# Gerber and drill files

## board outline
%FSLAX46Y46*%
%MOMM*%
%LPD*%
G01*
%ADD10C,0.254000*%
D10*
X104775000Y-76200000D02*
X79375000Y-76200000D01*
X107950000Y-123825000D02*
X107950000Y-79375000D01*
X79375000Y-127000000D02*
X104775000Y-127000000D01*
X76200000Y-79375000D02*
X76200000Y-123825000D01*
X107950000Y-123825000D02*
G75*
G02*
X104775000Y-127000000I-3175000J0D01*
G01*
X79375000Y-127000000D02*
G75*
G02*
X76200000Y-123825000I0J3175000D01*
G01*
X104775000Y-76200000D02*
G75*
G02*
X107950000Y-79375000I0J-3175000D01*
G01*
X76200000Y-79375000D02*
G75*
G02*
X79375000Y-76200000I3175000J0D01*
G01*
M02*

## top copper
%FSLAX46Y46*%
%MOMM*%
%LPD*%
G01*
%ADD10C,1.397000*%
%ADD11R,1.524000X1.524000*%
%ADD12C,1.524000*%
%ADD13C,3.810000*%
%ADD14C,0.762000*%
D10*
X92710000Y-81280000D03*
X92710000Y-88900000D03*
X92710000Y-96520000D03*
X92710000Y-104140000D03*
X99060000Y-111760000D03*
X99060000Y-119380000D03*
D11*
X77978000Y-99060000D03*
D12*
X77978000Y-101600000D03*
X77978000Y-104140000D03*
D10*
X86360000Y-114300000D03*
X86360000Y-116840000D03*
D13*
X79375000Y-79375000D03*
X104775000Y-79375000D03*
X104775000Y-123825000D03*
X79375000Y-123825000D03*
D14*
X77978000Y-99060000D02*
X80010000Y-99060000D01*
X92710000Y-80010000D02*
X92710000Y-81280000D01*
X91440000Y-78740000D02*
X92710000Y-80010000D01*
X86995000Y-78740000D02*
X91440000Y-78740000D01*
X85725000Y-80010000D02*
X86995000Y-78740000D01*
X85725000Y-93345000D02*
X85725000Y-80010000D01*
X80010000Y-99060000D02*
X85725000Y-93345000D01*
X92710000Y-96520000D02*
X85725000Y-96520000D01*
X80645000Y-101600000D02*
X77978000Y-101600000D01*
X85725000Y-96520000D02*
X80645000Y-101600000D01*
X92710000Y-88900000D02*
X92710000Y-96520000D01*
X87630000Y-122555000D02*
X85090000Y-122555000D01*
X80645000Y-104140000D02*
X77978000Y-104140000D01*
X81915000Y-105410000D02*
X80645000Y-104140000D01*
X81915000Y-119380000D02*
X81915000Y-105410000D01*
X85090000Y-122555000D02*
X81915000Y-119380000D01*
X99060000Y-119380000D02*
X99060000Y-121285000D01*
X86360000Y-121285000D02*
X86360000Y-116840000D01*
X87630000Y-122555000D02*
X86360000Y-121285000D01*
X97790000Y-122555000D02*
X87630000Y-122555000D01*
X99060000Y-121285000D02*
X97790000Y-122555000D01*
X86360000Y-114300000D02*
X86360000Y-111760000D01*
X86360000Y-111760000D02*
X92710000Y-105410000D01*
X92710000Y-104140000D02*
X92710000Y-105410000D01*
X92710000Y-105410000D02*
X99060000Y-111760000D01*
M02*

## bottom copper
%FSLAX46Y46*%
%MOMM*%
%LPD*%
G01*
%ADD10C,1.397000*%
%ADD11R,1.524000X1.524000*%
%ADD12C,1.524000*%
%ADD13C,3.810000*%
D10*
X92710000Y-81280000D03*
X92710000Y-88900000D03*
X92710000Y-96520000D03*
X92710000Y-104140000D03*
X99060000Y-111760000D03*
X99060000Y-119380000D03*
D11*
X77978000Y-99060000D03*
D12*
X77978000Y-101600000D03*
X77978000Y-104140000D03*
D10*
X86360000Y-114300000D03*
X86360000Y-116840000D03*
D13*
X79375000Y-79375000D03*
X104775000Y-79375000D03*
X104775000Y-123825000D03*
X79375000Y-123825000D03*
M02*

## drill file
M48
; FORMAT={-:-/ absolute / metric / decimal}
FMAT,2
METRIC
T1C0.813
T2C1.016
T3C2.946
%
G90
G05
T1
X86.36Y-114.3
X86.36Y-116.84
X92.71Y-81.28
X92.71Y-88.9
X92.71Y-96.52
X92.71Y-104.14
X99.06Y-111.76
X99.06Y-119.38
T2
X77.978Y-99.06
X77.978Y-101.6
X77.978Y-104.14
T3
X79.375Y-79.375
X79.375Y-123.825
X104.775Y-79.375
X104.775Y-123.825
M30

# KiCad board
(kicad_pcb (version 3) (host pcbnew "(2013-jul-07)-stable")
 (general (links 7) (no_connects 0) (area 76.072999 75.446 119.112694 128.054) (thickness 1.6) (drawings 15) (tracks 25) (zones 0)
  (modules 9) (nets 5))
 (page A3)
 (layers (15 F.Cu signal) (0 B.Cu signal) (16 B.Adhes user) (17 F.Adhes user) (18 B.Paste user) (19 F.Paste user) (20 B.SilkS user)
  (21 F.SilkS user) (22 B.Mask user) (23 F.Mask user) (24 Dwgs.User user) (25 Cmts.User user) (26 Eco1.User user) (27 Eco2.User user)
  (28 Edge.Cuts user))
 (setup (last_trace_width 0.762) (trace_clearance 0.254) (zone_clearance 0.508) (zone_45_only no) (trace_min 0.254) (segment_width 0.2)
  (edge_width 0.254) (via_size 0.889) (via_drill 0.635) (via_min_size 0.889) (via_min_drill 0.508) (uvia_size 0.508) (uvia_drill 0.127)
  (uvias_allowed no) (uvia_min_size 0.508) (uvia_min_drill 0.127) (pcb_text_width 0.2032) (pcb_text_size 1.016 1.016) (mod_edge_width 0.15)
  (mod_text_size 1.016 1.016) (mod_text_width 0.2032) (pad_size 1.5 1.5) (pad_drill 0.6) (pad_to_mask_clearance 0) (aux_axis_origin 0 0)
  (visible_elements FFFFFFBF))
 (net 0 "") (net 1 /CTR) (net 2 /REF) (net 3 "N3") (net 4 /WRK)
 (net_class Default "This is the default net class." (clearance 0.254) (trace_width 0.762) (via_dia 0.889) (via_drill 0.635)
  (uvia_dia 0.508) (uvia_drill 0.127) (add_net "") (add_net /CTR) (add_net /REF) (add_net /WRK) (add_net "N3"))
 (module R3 (layer F.Cu) (at 92.71 85.09 270) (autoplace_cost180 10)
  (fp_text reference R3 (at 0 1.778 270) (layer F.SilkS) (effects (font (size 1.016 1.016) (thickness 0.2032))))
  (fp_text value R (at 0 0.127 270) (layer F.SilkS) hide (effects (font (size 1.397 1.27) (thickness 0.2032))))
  (pad 1 thru_hole circle (at -3.81 0 270) (size 1.397 1.397) (drill 0.8128) (layers *.Cu *.Mask F.SilkS) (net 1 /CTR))
  (pad 2 thru_hole circle (at 3.81 0 270) (size 1.397 1.397) (drill 0.8128) (layers *.Cu *.Mask F.SilkS) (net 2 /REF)))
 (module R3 (layer F.Cu) (at 92.71 100.33 270) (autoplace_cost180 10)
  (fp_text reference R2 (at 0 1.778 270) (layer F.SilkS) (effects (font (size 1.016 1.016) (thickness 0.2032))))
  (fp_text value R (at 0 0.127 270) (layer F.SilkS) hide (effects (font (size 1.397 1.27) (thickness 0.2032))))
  (pad 1 thru_hole circle (at -3.81 0 270) (size 1.397 1.397) (drill 0.8128) (layers *.Cu *.Mask F.SilkS) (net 2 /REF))
  (pad 2 thru_hole circle (at 3.81 0 270) (size 1.397 1.397) (drill 0.8128) (layers *.Cu *.Mask F.SilkS) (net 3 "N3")))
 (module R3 (layer F.Cu) (at 99.06 115.57 270) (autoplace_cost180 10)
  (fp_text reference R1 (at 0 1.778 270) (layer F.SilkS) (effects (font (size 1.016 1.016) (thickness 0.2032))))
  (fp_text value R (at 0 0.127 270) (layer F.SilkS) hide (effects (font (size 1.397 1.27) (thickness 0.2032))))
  (pad 1 thru_hole circle (at -3.81 0 270) (size 1.397 1.397) (drill 0.8128) (layers *.Cu *.Mask F.SilkS) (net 3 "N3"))
  (pad 2 thru_hole circle (at 3.81 0 270) (size 1.397 1.397) (drill 0.8128) (layers *.Cu *.Mask F.SilkS) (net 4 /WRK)))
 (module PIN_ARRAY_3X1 (layer F.Cu) (at 77.978 101.6 270)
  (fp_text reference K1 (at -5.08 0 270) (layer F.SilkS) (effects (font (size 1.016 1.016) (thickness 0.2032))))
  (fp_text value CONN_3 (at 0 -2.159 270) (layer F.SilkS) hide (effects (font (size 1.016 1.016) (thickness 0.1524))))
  (pad 1 thru_hole rect (at -2.54 0 270) (size 1.524 1.524) (drill 1.016) (layers *.Cu *.Mask F.SilkS) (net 1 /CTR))
  (pad 2 thru_hole circle (at 0 0 270) (size 1.524 1.524) (drill 1.016) (layers *.Cu *.Mask F.SilkS) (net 2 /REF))
  (pad 3 thru_hole circle (at 2.54 0 270) (size 1.524 1.524) (drill 1.016) (layers *.Cu *.Mask F.SilkS) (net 4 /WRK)))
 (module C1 (layer F.Cu) (at 86.36 115.57 270)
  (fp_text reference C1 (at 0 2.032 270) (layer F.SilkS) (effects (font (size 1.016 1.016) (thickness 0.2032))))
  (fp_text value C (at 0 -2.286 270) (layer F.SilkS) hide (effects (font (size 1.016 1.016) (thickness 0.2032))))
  (pad 1 thru_hole circle (at -1.27 0 270) (size 1.397 1.397) (drill 0.8128) (layers *.Cu *.Mask F.SilkS) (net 3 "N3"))
  (pad 2 thru_hole circle (at 1.27 0 270) (size 1.397 1.397) (drill 0.8128) (layers *.Cu *.Mask F.SilkS) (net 4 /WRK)))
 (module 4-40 (layer F.Cu) (at 79.375 79.375)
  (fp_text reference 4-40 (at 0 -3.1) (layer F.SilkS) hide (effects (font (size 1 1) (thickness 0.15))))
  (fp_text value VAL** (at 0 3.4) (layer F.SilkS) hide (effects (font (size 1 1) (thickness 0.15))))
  (pad "" thru_hole circle (at 0 0) (size 3.81 3.81) (drill 2.9464) (layers *.Cu *.Mask F.SilkS)))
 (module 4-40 (layer F.Cu) (at 104.775 79.375)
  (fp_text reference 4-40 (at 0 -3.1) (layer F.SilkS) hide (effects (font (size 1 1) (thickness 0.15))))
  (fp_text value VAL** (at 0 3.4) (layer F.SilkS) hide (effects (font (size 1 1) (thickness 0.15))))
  (pad "" thru_hole circle (at 0 0) (size 3.81 3.81) (drill 2.9464) (layers *.Cu *.Mask F.SilkS)))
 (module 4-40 (layer F.Cu) (at 104.775 123.825)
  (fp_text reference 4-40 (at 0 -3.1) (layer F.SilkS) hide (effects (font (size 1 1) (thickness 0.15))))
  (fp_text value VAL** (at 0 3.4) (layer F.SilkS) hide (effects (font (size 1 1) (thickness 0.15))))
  (pad "" thru_hole circle (at 0 0) (size 3.81 3.81) (drill 2.9464) (layers *.Cu *.Mask F.SilkS)))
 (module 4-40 (layer F.Cu) (at 79.375 123.825)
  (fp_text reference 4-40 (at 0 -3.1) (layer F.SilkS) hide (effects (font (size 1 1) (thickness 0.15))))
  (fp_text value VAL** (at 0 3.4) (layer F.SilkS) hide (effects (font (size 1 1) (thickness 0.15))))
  (pad "" thru_hole circle (at 0 0) (size 3.81 3.81) (drill 2.9464) (layers *.Cu *.Mask F.SilkS)))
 (gr_line (start 104.775 76.2) (end 79.375 76.2) (angle 90) (layer Edge.Cuts) (width 0.254))
 (gr_line (start 107.95 123.825) (end 107.95 79.375) (angle 90) (layer Edge.Cuts) (width 0.254))
 (gr_line (start 79.375 127) (end 104.775 127) (angle 90) (layer Edge.Cuts) (width 0.254))
 (gr_line (start 76.2 79.375) (end 76.2 123.825) (angle 90) (layer Edge.Cuts) (width 0.254))
 (gr_arc (start 104.775 123.825) (end 107.95 123.825) (angle 90) (layer Edge.Cuts) (width 0.254))
 (gr_arc (start 79.375 123.825) (end 79.375 127) (angle 90) (layer Edge.Cuts) (width 0.254))
 (gr_arc (start 104.775 79.375) (end 104.775 76.2) (angle 90) (layer Edge.Cuts) (width 0.254))
 (gr_arc (start 79.375 79.375) (end 76.2 79.375) (angle 90) (layer Edge.Cuts) (width 0.254))
 (segment (start 77.978 99.06) (end 80.01 99.06) (width 0.762) (layer F.Cu) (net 1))
 (segment (start 92.71 80.01) (end 92.71 81.28) (width 0.762) (layer F.Cu) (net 1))
 (segment (start 91.44 78.74) (end 92.71 80.01) (width 0.762) (layer F.Cu) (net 1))
 (segment (start 86.995 78.74) (end 91.44 78.74) (width 0.762) (layer F.Cu) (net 1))
 (segment (start 85.725 80.01) (end 86.995 78.74) (width 0.762) (layer F.Cu) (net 1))
 (segment (start 85.725 93.345) (end 85.725 80.01) (width 0.762) (layer F.Cu) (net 1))
 (segment (start 80.01 99.06) (end 85.725 93.345) (width 0.762) (layer F.Cu) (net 1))
 (segment (start 92.71 96.52) (end 85.725 96.52) (width 0.762) (layer F.Cu) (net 2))
 (segment (start 80.645 101.6) (end 77.978 101.6) (width 0.762) (layer F.Cu) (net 2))
 (segment (start 85.725 96.52) (end 80.645 101.6) (width 0.762) (layer F.Cu) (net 2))
 (segment (start 92.71 88.9) (end 92.71 96.52) (width 0.762) (layer F.Cu) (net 2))
 (segment (start 87.63 122.555) (end 85.09 122.555) (width 0.762) (layer F.Cu) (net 4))
 (segment (start 80.645 104.14) (end 77.978 104.14) (width 0.762) (layer F.Cu) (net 4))
 (segment (start 81.915 105.41) (end 80.645 104.14) (width 0.762) (layer F.Cu) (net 4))
 (segment (start 81.915 119.38) (end 81.915 105.41) (width 0.762) (layer F.Cu) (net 4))
 (segment (start 85.09 122.555) (end 81.915 119.38) (width 0.762) (layer F.Cu) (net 4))
 (segment (start 99.06 119.38) (end 99.06 121.285) (width 0.762) (layer F.Cu) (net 4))
 (segment (start 86.36 121.285) (end 86.36 116.84) (width 0.762) (layer F.Cu) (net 4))
 (segment (start 87.63 122.555) (end 86.36 121.285) (width 0.762) (layer F.Cu) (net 4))
 (segment (start 97.79 122.555) (end 87.63 122.555) (width 0.762) (layer F.Cu) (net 4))
 (segment (start 99.06 121.285) (end 97.79 122.555) (width 0.762) (layer F.Cu) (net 4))
 (segment (start 86.36 114.3) (end 86.36 111.76) (width 0.762) (layer F.Cu) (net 3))
 (segment (start 86.36 111.76) (end 92.71 105.41) (width 0.762) (layer F.Cu) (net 3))
 (segment (start 92.71 104.14) (end 92.71 105.41) (width 0.762) (layer F.Cu) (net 3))
 (segment (start 92.71 105.41) (end 99.06 111.76) (width 0.762) (layer F.Cu) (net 3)))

